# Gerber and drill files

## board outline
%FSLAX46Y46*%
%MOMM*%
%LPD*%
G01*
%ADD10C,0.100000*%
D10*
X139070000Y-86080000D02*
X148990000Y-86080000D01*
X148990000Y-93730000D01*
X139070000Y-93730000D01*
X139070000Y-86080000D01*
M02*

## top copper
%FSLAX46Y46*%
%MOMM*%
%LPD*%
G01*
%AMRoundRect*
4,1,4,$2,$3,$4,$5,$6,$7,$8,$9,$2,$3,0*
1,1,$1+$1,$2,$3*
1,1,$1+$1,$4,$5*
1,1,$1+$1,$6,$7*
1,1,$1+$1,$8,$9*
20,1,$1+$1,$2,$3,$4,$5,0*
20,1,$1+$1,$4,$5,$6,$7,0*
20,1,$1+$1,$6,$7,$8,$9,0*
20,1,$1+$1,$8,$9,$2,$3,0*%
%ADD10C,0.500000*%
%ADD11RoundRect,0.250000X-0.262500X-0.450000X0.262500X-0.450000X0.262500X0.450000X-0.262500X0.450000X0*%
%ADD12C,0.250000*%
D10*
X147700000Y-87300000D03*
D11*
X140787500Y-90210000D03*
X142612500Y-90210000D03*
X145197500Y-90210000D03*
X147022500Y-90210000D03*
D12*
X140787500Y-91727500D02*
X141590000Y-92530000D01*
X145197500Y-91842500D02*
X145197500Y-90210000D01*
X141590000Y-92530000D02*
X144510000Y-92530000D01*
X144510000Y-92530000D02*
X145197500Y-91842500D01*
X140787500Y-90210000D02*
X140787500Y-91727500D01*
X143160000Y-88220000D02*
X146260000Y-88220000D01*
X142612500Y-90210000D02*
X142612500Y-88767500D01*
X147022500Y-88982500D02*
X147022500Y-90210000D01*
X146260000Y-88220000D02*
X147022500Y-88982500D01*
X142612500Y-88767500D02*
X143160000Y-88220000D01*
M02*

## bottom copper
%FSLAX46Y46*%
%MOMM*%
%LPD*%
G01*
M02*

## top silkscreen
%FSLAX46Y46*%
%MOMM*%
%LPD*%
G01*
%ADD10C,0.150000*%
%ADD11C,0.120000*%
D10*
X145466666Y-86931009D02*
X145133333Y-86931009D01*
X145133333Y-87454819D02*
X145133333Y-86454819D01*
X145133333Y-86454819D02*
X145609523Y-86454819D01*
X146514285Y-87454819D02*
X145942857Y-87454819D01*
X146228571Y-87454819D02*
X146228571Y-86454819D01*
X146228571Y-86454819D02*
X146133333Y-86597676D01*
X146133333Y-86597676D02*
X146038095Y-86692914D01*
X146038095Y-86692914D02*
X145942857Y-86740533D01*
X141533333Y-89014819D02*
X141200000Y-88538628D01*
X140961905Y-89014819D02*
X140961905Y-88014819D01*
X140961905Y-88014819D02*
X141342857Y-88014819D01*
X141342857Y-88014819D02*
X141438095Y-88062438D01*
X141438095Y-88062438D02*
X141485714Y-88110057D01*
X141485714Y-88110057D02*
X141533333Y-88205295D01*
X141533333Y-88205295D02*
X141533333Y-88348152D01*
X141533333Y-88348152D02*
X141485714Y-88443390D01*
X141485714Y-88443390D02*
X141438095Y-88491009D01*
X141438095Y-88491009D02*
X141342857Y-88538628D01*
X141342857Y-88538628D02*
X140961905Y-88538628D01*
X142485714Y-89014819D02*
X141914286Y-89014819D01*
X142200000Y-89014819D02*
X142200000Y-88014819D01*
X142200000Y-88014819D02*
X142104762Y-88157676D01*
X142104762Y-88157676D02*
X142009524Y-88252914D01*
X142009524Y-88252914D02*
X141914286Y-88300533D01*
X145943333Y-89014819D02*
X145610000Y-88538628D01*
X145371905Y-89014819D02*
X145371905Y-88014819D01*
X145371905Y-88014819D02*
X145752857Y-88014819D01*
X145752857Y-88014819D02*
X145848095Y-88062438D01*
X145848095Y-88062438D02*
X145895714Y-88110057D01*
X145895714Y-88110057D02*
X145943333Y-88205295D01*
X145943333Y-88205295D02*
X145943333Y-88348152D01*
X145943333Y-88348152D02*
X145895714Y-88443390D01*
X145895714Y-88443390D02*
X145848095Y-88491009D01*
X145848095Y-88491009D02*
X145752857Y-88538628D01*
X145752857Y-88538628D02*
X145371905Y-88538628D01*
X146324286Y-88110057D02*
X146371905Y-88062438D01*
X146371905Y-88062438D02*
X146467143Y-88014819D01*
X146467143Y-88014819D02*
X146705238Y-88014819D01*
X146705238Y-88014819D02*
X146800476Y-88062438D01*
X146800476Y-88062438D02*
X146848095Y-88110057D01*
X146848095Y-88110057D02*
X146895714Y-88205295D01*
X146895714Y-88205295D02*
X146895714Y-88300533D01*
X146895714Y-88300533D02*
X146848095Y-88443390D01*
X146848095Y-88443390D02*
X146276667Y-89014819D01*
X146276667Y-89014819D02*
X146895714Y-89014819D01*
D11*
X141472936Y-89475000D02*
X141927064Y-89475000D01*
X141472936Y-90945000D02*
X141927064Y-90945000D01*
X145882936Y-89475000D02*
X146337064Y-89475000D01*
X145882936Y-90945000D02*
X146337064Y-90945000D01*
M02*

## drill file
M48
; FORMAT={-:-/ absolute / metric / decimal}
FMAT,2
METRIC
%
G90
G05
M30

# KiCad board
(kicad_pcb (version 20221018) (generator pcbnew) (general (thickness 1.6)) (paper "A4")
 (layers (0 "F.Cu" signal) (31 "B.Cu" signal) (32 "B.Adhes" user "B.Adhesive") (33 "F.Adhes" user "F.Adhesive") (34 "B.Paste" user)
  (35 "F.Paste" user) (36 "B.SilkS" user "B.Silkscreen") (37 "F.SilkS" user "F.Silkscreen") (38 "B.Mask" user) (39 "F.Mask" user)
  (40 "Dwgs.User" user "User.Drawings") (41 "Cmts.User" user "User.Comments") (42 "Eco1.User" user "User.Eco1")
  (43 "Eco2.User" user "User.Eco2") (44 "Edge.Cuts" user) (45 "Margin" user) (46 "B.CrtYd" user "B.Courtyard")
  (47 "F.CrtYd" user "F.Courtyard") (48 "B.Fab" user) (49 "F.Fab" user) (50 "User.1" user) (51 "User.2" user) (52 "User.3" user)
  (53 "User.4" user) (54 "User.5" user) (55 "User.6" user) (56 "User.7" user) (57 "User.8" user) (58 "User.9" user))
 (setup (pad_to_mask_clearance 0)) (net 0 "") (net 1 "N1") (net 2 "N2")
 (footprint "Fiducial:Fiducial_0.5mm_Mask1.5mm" (layer "F.Cu") (at 147.7 87.3)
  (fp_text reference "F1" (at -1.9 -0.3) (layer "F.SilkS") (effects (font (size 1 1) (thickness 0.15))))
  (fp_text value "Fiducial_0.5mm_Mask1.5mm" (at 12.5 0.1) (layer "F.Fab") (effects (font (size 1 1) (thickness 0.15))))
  (pad "" smd circle (at 0 0) (size 0.5 0.5) (layers "F.Cu" "F.Mask") (solder_mask_margin 0.5) (clearance 0.5)))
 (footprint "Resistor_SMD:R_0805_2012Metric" (layer "F.Cu") (at 141.7 90.21)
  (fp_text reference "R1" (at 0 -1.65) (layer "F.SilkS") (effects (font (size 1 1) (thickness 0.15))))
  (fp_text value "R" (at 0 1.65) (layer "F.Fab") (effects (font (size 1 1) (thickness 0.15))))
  (fp_line (start -0.227064 -0.735) (end 0.227064 -0.735) (stroke (width 0.12) (type solid)) (layer "F.SilkS"))
  (fp_line (start -0.227064 0.735) (end 0.227064 0.735) (stroke (width 0.12) (type solid)) (layer "F.SilkS"))
  (pad "1" smd roundrect (at -0.9125 0) (size 1.025 1.4) (layers "F.Cu" "F.Paste" "F.Mask") (roundrect_rratio 0.243902) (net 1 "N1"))
  (pad "2" smd roundrect (at 0.9125 0) (size 1.025 1.4) (layers "F.Cu" "F.Paste" "F.Mask") (roundrect_rratio 0.243902) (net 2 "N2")))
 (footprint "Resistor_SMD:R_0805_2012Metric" (layer "F.Cu") (at 146.11 90.21)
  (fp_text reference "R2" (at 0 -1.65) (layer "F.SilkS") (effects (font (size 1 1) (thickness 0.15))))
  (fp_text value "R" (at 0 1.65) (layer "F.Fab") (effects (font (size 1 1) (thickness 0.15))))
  (fp_line (start -0.227064 -0.735) (end 0.227064 -0.735) (stroke (width 0.12) (type solid)) (layer "F.SilkS"))
  (fp_line (start -0.227064 0.735) (end 0.227064 0.735) (stroke (width 0.12) (type solid)) (layer "F.SilkS"))
  (pad "1" smd roundrect (at -0.9125 0) (size 1.025 1.4) (layers "F.Cu" "F.Paste" "F.Mask") (roundrect_rratio 0.243902) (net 1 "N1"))
  (pad "2" smd roundrect (at 0.9125 0) (size 1.025 1.4) (layers "F.Cu" "F.Paste" "F.Mask") (roundrect_rratio 0.243902) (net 2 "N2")))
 (gr_rect (start 139.07 86.08) (end 148.99 93.73) (stroke (width 0.1) (type solid)) (fill none) (layer "Edge.Cuts"))
 (segment (start 140.7875 91.7275) (end 141.59 92.53) (width 0.25) (layer "F.Cu") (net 1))
 (segment (start 145.1975 91.8425) (end 145.1975 90.21) (width 0.25) (layer "F.Cu") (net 1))
 (segment (start 141.59 92.53) (end 144.51 92.53) (width 0.25) (layer "F.Cu") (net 1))
 (segment (start 144.51 92.53) (end 145.1975 91.8425) (width 0.25) (layer "F.Cu") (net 1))
 (segment (start 140.7875 90.21) (end 140.7875 91.7275) (width 0.25) (layer "F.Cu") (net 1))
 (segment (start 143.16 88.22) (end 146.26 88.22) (width 0.25) (layer "F.Cu") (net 2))
 (segment (start 142.6125 90.21) (end 142.6125 88.7675) (width 0.25) (layer "F.Cu") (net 2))
 (segment (start 147.0225 88.9825) (end 147.0225 90.21) (width 0.25) (layer "F.Cu") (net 2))
 (segment (start 146.26 88.22) (end 147.0225 88.9825) (width 0.25) (layer "F.Cu") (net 2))
 (segment (start 142.6125 88.7675) (end 143.16 88.22) (width 0.25) (layer "F.Cu") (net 2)))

